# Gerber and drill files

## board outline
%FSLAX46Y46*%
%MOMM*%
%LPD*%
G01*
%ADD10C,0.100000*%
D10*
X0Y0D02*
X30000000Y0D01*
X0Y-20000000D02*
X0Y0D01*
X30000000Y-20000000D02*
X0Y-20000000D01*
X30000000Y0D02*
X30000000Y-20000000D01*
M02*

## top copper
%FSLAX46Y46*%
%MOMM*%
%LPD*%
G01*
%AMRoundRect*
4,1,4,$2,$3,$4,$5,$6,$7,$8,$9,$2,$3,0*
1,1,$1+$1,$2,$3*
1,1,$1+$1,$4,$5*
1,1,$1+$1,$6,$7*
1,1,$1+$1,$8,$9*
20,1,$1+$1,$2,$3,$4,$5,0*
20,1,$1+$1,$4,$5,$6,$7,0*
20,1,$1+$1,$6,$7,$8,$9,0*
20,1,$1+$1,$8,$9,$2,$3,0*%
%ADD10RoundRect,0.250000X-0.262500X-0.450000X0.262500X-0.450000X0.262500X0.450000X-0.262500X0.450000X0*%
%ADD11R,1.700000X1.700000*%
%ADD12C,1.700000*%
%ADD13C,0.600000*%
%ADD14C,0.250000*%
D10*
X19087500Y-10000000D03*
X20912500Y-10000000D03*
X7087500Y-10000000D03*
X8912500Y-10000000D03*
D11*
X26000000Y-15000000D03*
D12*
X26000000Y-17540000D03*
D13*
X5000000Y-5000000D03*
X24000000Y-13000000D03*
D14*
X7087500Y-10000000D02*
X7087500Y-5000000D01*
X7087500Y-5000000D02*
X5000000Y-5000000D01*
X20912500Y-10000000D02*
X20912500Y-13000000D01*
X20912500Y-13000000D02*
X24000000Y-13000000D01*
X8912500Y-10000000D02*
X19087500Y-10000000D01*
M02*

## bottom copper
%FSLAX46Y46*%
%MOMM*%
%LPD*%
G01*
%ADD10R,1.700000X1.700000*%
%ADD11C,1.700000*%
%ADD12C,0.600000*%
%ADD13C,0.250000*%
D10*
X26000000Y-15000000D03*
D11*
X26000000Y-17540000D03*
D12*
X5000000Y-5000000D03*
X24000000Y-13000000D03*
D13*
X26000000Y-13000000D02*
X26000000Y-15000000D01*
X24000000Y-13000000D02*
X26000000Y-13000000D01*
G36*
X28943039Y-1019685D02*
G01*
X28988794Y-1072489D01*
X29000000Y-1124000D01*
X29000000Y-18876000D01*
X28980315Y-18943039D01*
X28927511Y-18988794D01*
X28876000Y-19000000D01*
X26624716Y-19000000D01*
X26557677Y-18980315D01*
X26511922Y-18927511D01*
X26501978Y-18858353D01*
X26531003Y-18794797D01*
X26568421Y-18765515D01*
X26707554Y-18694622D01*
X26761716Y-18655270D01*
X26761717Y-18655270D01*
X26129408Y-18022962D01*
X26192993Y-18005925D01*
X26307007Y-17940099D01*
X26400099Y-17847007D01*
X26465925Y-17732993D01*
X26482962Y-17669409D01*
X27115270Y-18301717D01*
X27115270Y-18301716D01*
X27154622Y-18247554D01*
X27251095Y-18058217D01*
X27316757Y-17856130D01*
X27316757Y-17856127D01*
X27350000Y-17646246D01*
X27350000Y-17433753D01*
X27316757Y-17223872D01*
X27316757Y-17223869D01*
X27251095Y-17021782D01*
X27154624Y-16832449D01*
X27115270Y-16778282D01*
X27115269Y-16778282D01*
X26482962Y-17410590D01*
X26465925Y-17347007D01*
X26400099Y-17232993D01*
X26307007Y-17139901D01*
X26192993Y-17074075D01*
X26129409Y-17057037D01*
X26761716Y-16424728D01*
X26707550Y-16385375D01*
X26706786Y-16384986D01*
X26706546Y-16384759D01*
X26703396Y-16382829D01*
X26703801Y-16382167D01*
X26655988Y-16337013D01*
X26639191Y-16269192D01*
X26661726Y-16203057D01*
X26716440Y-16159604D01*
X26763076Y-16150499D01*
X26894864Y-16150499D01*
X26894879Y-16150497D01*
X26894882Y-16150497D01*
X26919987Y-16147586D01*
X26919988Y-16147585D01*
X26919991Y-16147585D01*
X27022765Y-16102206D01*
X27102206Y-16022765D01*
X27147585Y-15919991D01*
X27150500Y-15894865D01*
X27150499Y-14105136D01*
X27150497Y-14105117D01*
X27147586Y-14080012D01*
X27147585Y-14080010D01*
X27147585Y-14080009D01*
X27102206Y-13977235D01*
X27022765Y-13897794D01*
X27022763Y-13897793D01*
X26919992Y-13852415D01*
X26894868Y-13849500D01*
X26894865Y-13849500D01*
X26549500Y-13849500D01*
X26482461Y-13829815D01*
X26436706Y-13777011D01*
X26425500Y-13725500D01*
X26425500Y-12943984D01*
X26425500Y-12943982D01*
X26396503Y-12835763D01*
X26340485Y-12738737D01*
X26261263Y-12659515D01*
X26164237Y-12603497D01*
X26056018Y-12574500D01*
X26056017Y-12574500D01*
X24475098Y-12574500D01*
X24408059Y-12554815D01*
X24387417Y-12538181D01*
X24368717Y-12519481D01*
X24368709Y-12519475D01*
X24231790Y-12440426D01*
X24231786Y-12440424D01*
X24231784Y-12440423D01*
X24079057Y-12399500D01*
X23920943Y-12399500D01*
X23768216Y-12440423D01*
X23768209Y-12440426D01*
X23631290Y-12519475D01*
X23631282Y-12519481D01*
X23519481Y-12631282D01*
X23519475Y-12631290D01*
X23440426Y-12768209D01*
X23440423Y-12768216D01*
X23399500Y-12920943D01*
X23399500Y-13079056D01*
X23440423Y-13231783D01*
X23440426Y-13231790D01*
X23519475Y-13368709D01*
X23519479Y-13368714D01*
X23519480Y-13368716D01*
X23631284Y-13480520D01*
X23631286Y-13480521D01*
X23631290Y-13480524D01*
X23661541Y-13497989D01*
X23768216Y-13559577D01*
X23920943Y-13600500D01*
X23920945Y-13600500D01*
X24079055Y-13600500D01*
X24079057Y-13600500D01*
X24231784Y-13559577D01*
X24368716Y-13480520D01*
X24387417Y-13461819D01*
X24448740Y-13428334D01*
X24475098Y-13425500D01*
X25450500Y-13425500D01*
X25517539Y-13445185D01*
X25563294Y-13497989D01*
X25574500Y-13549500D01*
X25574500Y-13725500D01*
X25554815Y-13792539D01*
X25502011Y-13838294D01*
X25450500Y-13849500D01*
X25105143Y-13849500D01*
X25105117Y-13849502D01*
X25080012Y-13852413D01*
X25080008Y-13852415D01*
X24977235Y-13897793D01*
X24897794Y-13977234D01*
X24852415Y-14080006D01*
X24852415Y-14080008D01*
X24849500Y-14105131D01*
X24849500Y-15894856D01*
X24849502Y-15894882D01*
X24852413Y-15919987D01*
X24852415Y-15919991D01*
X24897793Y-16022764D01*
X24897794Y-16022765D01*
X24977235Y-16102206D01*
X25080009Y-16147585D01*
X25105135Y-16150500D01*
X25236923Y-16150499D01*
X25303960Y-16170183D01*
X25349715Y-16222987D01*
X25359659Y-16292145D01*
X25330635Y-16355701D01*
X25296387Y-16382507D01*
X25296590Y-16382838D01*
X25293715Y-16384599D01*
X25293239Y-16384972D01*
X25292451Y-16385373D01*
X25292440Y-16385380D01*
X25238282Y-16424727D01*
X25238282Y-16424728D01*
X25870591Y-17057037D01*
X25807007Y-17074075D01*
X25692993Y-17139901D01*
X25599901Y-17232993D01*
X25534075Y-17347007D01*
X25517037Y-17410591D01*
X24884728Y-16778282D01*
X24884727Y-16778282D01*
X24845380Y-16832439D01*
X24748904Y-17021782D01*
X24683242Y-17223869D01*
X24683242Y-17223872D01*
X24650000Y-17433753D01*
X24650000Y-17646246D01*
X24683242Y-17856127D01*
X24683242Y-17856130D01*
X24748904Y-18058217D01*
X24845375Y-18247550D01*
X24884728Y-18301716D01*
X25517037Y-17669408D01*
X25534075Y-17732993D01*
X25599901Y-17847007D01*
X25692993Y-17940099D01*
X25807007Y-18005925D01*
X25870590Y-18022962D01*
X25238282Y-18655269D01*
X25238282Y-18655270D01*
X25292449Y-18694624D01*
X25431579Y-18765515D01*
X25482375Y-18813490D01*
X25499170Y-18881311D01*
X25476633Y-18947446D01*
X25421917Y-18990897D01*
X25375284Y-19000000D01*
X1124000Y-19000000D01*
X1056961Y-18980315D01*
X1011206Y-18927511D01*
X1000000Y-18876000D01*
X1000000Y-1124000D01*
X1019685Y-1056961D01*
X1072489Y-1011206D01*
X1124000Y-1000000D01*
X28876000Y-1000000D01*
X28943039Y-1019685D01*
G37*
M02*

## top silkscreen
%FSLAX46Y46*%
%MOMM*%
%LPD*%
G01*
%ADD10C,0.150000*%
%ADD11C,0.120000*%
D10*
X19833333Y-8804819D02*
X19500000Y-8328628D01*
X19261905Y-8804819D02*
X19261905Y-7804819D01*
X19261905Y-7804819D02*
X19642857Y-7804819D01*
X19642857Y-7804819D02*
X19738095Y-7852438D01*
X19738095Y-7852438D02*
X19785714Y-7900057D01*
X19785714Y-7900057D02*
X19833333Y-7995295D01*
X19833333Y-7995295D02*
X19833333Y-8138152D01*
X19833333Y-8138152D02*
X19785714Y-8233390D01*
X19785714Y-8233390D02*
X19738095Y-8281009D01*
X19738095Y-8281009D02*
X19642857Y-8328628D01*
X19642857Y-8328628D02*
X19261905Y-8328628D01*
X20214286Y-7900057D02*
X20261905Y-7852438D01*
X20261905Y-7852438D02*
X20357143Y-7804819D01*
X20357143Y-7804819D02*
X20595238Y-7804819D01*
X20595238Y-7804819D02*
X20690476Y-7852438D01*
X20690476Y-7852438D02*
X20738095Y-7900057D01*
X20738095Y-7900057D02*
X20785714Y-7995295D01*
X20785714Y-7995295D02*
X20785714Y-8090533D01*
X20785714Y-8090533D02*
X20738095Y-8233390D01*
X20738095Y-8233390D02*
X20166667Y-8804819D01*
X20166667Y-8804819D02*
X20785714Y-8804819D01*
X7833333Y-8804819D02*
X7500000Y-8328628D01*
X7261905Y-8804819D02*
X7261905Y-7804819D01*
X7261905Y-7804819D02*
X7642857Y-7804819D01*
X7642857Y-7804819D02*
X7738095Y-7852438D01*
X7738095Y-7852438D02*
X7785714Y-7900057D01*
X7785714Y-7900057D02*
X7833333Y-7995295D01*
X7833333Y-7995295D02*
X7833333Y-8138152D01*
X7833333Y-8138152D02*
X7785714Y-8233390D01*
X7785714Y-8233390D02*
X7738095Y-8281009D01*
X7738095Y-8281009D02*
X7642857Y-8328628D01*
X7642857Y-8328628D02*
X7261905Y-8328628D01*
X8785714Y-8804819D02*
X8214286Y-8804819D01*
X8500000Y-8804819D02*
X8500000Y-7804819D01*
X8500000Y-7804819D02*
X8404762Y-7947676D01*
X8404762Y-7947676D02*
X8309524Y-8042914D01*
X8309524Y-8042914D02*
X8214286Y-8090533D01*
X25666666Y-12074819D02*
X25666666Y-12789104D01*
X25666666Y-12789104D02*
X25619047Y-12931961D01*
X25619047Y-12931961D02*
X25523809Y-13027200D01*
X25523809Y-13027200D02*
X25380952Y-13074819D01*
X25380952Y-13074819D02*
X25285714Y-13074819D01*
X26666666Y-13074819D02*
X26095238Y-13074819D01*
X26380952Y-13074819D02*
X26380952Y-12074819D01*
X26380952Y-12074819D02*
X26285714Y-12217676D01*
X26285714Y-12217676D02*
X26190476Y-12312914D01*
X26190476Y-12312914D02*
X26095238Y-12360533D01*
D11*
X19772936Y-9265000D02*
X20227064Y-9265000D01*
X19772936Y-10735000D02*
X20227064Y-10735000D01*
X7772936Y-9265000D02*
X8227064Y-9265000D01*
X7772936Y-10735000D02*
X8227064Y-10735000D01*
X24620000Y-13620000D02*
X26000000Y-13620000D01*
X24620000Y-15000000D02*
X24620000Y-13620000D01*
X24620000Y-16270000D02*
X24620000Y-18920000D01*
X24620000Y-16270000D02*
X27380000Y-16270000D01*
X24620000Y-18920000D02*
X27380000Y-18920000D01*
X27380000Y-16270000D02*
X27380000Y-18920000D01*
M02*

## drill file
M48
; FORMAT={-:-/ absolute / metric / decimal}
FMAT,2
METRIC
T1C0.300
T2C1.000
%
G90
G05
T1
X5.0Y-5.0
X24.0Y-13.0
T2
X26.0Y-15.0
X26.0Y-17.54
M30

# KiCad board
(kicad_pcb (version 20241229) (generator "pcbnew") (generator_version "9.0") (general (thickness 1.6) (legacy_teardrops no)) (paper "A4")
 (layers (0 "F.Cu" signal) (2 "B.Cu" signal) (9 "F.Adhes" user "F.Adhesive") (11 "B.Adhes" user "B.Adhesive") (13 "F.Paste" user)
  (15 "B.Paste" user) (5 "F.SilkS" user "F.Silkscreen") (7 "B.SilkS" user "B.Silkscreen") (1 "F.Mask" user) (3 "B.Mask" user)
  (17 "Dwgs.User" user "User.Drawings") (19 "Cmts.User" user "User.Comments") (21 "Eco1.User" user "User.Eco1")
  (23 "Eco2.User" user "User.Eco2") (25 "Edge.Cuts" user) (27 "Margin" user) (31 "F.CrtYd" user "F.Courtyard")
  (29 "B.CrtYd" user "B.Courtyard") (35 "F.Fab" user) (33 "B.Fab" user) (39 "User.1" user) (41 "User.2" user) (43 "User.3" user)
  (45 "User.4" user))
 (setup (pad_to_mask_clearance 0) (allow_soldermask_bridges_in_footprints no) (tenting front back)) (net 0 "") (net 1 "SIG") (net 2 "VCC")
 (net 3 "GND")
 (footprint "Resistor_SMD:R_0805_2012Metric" (layer "F.Cu") (at 20 10)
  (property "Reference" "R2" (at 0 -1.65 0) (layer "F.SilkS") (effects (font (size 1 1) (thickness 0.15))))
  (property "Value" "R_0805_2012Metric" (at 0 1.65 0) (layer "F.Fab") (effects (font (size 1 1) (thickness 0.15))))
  (fp_line (start -0.227064 -0.735) (end 0.227064 -0.735) (stroke (width 0.12) (type solid)) (layer "F.SilkS"))
  (fp_line (start -0.227064 0.735) (end 0.227064 0.735) (stroke (width 0.12) (type solid)) (layer "F.SilkS"))
  (pad "1" smd roundrect (at -0.9125 0) (size 1.025 1.4) (layers "F.Cu" "F.Mask" "F.Paste") (roundrect_rratio 0.243902) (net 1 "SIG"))
  (pad "2" smd roundrect (at 0.9125 0) (size 1.025 1.4) (layers "F.Cu" "F.Mask" "F.Paste") (roundrect_rratio 0.243902) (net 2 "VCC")))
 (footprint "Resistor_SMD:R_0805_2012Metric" (layer "F.Cu") (at 8 10)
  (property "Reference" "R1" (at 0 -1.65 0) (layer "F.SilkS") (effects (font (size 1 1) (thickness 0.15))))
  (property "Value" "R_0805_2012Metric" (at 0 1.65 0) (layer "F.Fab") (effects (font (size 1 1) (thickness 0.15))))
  (fp_line (start -0.227064 -0.735) (end 0.227064 -0.735) (stroke (width 0.12) (type solid)) (layer "F.SilkS"))
  (fp_line (start -0.227064 0.735) (end 0.227064 0.735) (stroke (width 0.12) (type solid)) (layer "F.SilkS"))
  (pad "1" smd roundrect (at -0.9125 0) (size 1.025 1.4) (layers "F.Cu" "F.Mask" "F.Paste") (roundrect_rratio 0.243902) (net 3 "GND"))
  (pad "2" smd roundrect (at 0.9125 0) (size 1.025 1.4) (layers "F.Cu" "F.Mask" "F.Paste") (roundrect_rratio 0.243902) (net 1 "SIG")))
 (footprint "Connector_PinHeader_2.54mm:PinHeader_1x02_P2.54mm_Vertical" (layer "F.Cu") (at 26 15)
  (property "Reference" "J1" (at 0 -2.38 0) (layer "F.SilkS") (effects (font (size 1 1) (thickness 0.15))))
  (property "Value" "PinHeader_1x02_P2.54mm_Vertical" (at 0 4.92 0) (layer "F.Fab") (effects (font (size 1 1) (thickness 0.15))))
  (fp_line (start -1.38 -1.38) (end 0 -1.38) (stroke (width 0.12) (type solid)) (layer "F.SilkS"))
  (fp_line (start -1.38 0) (end -1.38 -1.38) (stroke (width 0.12) (type solid)) (layer "F.SilkS"))
  (fp_line (start -1.38 1.27) (end -1.38 3.92) (stroke (width 0.12) (type solid)) (layer "F.SilkS"))
  (fp_line (start -1.38 1.27) (end 1.38 1.27) (stroke (width 0.12) (type solid)) (layer "F.SilkS"))
  (fp_line (start -1.38 3.92) (end 1.38 3.92) (stroke (width 0.12) (type solid)) (layer "F.SilkS"))
  (fp_line (start 1.38 1.27) (end 1.38 3.92) (stroke (width 0.12) (type solid)) (layer "F.SilkS"))
  (pad "1" thru_hole rect (at 0 0) (size 1.7 1.7) (drill 1) (layers "*.Cu" "*.Mask") (remove_unused_layers no) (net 2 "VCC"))
  (pad "2" thru_hole circle (at 0 2.54) (size 1.7 1.7) (drill 1) (layers "*.Cu" "*.Mask") (remove_unused_layers no) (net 3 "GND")))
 (gr_line (start 0 0) (end 30 0) (stroke (width 0.1) (type default)) (layer "Edge.Cuts"))
 (gr_line (start 0 20) (end 0 0) (stroke (width 0.1) (type default)) (layer "Edge.Cuts"))
 (gr_line (start 30 20) (end 0 20) (stroke (width 0.1) (type default)) (layer "Edge.Cuts"))
 (gr_line (start 30 0) (end 30 20) (stroke (width 0.1) (type default)) (layer "Edge.Cuts"))
 (segment (start 7.0875 10) (end 7.0875 5) (width 0.25) (layer "F.Cu") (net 3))
 (segment (start 7.0875 5) (end 5 5) (width 0.25) (layer "F.Cu") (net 3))
 (via (at 5 5) (size 0.6) (drill 0.3) (layers "F.Cu" "B.Cu") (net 3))
 (segment (start 20.9125 10) (end 20.9125 13) (width 0.25) (layer "F.Cu") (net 2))
 (segment (start 20.9125 13) (end 24 13) (width 0.25) (layer "F.Cu") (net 2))
 (via (at 24 13) (size 0.6) (drill 0.3) (layers "F.Cu" "B.Cu") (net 2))
 (segment (start 26 13) (end 26 15) (width 0.25) (layer "B.Cu") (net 2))
 (segment (start 24 13) (end 26 13) (width 0.25) (layer "B.Cu") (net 2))
 (segment (start 8.9125 10) (end 19.0875 10) (width 0.25) (layer "F.Cu") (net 1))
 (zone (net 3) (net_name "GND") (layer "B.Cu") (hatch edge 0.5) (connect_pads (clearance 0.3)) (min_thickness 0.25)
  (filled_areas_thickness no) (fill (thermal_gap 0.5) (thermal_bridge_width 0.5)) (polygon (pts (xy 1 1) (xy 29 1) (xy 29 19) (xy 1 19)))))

